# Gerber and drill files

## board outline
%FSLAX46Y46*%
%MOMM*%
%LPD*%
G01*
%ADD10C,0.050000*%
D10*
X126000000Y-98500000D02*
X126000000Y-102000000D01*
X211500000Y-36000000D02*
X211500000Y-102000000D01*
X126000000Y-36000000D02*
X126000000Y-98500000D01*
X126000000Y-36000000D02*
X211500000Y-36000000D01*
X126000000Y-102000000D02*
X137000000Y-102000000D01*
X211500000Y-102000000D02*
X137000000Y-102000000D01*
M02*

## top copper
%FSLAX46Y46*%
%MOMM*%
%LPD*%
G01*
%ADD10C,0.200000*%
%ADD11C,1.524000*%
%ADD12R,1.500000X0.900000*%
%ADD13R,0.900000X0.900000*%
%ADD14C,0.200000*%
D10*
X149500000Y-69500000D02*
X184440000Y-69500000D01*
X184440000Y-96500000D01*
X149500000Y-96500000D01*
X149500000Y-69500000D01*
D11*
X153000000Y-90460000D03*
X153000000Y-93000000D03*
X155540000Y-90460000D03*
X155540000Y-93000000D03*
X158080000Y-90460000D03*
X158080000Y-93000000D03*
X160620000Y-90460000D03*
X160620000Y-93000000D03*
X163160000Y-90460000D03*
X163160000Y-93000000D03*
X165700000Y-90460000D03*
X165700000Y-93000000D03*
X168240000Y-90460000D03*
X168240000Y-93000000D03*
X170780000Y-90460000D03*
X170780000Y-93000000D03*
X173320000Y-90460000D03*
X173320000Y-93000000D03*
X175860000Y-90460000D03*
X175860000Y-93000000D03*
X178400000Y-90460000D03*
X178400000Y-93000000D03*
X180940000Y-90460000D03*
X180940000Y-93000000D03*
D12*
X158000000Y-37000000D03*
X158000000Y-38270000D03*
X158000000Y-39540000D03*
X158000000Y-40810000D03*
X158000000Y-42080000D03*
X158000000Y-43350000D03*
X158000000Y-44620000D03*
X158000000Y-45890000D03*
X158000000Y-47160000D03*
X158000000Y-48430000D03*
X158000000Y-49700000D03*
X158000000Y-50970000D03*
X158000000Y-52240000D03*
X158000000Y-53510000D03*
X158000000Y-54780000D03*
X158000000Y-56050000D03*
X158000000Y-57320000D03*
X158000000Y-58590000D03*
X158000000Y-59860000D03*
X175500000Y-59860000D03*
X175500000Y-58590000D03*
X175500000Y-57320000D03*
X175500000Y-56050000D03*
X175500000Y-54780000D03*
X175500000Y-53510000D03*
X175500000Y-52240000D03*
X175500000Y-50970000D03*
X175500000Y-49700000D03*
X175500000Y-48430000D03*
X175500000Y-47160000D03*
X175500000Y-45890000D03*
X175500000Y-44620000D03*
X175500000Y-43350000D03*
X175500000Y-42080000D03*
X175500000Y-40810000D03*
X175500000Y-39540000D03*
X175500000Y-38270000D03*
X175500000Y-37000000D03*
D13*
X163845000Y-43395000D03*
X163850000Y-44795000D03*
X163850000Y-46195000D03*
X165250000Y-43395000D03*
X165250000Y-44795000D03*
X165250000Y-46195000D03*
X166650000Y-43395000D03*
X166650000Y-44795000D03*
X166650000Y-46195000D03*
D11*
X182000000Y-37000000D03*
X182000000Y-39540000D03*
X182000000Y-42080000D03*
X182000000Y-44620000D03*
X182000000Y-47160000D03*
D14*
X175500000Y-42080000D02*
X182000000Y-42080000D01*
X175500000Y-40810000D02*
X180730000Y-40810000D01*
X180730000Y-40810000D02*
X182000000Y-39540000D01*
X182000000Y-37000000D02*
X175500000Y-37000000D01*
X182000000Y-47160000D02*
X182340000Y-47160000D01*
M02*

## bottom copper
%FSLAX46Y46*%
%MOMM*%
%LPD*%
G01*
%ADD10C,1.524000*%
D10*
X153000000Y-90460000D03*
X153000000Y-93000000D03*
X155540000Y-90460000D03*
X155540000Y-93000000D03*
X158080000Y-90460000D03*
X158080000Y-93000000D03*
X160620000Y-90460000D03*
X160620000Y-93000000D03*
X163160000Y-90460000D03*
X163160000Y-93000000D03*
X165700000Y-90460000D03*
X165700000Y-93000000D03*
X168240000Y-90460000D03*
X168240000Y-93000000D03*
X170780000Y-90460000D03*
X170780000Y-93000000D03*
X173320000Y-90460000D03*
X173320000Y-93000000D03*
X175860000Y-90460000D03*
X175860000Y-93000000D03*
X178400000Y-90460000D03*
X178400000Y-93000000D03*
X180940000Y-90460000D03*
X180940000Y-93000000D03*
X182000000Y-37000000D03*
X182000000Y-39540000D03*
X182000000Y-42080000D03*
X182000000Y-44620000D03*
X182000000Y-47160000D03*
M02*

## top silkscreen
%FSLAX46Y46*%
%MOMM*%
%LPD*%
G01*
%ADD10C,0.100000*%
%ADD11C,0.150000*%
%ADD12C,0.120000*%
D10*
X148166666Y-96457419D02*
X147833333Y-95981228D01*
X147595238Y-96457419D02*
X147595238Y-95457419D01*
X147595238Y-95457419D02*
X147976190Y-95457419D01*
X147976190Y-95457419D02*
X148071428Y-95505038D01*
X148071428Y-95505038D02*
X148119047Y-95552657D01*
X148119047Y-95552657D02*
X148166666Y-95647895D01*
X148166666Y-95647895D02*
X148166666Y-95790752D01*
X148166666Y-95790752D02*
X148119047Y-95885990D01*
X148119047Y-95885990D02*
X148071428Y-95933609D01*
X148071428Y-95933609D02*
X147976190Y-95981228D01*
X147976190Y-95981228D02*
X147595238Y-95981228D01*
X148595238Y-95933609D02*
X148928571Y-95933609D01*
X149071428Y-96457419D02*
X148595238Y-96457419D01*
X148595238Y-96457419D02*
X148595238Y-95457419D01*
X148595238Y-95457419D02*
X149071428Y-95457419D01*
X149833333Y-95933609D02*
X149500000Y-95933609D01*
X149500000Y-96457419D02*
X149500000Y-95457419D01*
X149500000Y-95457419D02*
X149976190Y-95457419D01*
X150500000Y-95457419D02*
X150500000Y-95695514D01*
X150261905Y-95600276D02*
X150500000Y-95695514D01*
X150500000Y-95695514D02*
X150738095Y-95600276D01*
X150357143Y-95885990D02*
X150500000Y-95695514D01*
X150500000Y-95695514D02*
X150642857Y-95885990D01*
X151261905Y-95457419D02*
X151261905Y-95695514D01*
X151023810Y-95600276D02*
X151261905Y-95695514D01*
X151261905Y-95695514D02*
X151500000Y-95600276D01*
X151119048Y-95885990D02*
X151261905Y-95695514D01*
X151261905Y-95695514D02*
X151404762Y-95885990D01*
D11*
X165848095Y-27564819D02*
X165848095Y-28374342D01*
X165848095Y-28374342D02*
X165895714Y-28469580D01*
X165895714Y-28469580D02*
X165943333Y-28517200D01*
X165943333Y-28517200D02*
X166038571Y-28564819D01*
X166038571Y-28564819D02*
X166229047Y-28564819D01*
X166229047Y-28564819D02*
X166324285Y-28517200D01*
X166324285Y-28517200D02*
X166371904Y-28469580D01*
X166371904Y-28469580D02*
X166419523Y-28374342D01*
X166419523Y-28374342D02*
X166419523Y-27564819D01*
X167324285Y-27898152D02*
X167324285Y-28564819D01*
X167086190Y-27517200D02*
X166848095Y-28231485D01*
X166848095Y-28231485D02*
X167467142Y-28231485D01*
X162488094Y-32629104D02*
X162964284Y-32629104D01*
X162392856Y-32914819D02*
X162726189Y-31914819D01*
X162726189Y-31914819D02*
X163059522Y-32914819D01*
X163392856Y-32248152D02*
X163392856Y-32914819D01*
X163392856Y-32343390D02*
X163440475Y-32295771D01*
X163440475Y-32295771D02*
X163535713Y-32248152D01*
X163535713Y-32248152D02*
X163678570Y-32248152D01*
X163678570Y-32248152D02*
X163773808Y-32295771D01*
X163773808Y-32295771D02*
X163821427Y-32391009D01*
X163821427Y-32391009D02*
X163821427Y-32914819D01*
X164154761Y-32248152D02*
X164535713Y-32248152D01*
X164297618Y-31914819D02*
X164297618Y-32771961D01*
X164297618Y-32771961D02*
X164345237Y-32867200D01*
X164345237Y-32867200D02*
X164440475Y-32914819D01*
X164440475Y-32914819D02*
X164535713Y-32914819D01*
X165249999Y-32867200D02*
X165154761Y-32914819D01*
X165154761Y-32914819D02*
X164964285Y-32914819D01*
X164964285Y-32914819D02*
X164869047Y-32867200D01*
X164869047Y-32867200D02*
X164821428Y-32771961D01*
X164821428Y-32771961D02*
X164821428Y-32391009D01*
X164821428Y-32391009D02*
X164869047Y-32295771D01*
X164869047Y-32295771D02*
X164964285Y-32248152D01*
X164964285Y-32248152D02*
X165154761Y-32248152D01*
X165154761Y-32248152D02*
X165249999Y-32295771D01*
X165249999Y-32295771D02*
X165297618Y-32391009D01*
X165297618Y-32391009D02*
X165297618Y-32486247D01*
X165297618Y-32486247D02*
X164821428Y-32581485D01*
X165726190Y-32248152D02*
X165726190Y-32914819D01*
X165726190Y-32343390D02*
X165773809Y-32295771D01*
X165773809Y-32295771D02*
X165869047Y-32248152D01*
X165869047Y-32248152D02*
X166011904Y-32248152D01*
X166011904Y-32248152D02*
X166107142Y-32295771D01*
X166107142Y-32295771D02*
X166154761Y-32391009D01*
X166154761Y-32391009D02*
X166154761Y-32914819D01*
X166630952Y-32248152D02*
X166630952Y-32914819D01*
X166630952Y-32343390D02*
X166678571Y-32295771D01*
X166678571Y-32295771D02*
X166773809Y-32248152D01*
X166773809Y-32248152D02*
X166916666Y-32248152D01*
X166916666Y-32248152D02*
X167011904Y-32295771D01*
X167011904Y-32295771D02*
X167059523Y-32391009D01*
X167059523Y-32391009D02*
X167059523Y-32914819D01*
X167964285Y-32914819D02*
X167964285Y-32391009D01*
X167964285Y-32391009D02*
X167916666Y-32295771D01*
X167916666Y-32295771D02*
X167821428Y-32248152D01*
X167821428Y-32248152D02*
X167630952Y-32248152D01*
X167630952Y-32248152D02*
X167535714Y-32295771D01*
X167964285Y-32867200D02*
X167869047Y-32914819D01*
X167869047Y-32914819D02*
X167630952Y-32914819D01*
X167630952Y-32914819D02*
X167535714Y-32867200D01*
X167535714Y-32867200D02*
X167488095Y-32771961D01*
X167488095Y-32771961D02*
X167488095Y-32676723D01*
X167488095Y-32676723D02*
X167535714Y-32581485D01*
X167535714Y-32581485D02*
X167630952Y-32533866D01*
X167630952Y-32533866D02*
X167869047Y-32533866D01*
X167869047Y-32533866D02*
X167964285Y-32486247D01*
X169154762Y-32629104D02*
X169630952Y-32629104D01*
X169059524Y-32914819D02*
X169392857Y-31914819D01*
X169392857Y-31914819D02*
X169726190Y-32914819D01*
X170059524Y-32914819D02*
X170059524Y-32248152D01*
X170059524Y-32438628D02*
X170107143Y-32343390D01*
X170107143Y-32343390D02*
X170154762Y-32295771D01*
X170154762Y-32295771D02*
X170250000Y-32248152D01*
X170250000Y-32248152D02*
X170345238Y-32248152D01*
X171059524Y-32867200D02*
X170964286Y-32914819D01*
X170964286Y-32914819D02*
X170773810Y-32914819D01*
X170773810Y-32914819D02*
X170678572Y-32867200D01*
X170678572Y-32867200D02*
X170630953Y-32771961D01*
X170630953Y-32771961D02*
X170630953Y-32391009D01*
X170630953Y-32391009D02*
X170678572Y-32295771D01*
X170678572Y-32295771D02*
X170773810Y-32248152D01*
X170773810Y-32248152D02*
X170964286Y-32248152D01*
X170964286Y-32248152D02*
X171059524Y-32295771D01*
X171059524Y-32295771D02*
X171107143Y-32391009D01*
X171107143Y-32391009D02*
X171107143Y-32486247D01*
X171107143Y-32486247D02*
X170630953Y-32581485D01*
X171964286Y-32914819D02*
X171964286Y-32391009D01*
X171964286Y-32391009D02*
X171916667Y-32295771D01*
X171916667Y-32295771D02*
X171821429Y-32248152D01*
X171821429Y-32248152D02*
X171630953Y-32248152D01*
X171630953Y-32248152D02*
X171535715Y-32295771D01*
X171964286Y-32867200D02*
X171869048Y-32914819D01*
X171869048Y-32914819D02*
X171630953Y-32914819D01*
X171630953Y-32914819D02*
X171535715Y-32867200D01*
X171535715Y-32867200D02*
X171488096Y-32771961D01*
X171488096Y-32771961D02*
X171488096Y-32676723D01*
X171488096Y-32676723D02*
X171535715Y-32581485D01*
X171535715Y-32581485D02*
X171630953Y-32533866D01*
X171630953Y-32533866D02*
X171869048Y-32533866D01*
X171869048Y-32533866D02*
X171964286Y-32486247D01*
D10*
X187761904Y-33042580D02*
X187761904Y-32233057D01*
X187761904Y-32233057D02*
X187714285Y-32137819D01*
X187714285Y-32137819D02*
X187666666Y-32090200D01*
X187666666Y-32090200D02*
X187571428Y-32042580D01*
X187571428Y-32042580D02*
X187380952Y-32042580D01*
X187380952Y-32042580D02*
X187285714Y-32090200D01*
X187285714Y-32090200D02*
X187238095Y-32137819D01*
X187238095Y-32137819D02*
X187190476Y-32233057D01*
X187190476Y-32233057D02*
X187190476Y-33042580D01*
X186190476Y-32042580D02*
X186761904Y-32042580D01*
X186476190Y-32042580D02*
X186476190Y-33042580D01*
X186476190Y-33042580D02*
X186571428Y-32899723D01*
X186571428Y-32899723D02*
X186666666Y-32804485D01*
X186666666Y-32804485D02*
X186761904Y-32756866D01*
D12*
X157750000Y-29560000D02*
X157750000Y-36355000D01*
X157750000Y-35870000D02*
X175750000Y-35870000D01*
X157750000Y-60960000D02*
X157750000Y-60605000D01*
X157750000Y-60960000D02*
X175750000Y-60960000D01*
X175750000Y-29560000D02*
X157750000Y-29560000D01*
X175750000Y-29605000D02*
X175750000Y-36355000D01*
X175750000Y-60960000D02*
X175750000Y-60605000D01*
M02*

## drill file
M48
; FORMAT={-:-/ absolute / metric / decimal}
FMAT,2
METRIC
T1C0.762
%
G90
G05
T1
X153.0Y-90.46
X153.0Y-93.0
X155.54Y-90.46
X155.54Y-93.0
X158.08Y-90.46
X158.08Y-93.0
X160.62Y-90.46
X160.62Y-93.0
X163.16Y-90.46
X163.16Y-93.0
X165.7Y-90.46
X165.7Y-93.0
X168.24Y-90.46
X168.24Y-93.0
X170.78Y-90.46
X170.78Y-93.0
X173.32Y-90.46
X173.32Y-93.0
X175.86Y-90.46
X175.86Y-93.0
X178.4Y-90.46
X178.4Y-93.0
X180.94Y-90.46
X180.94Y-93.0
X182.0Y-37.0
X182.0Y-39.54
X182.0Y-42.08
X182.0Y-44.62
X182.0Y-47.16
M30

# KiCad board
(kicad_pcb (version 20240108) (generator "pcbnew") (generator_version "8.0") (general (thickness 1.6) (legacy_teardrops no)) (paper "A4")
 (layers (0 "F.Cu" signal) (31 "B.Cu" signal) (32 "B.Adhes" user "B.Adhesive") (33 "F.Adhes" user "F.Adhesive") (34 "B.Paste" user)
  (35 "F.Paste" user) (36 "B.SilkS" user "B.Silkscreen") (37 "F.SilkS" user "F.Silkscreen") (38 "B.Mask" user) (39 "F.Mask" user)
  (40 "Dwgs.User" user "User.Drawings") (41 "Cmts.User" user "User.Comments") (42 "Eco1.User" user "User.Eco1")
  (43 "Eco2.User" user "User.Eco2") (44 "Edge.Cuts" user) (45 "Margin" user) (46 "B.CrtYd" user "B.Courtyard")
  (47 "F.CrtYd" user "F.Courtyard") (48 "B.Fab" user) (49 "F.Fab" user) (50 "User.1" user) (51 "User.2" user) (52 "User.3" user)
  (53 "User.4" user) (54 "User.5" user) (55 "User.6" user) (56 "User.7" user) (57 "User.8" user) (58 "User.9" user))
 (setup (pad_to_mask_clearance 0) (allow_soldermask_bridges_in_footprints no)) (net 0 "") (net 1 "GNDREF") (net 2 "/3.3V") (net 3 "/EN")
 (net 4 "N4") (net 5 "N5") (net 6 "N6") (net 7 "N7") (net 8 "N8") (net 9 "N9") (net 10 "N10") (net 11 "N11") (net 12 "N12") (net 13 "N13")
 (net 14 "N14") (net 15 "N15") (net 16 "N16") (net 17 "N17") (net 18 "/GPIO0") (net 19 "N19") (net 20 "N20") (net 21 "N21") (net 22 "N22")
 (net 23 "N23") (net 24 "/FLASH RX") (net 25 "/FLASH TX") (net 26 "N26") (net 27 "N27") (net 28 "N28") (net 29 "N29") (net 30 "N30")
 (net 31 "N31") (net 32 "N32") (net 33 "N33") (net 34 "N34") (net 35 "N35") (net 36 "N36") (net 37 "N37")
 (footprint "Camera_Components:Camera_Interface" (layer "F.Cu") (at 149.5 96.5)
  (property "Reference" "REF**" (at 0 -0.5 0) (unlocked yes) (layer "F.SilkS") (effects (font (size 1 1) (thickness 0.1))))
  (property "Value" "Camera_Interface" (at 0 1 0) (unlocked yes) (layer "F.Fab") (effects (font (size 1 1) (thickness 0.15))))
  (fp_rect (start 0 0) (end 34.94 -27) (stroke (width 0.2) (type default)) (fill none) (layer "F.Cu"))
  (pad "1" thru_hole circle (at 3.5 -6.04 270) (size 1.524 1.524) (drill 0.762) (layers "*.Cu" "*.Mask") (remove_unused_layers no))
  (pad "2" thru_hole circle (at 3.5 -3.5 270) (size 1.524 1.524) (drill 0.762) (layers "*.Cu" "*.Mask") (remove_unused_layers no))
  (pad "3" thru_hole circle (at 6.04 -6.04 270) (size 1.524 1.524) (drill 0.762) (layers "*.Cu" "*.Mask") (remove_unused_layers no))
  (pad "4" thru_hole circle (at 6.04 -3.5 270) (size 1.524 1.524) (drill 0.762) (layers "*.Cu" "*.Mask") (remove_unused_layers no))
  (pad "5" thru_hole circle (at 8.58 -6.04 270) (size 1.524 1.524) (drill 0.762) (layers "*.Cu" "*.Mask") (remove_unused_layers no))
  (pad "6" thru_hole circle (at 8.58 -3.5 270) (size 1.524 1.524) (drill 0.762) (layers "*.Cu" "*.Mask") (remove_unused_layers no))
  (pad "7" thru_hole circle (at 11.12 -6.04 270) (size 1.524 1.524) (drill 0.762) (layers "*.Cu" "*.Mask") (remove_unused_layers no))
  (pad "8" thru_hole circle (at 11.12 -3.5 270) (size 1.524 1.524) (drill 0.762) (layers "*.Cu" "*.Mask") (remove_unused_layers no))
  (pad "9" thru_hole circle (at 13.66 -6.04 270) (size 1.524 1.524) (drill 0.762) (layers "*.Cu" "*.Mask") (remove_unused_layers no))
  (pad "10" thru_hole circle (at 13.66 -3.5 270) (size 1.524 1.524) (drill 0.762) (layers "*.Cu" "*.Mask") (remove_unused_layers no))
  (pad "11" thru_hole circle (at 16.2 -6.04 270) (size 1.524 1.524) (drill 0.762) (layers "*.Cu" "*.Mask") (remove_unused_layers no))
  (pad "12" thru_hole circle (at 16.2 -3.5 270) (size 1.524 1.524) (drill 0.762) (layers "*.Cu" "*.Mask") (remove_unused_layers no))
  (pad "13" thru_hole circle (at 18.74 -6.04 270) (size 1.524 1.524) (drill 0.762) (layers "*.Cu" "*.Mask") (remove_unused_layers no))
  (pad "14" thru_hole circle (at 18.74 -3.5 270) (size 1.524 1.524) (drill 0.762) (layers "*.Cu" "*.Mask") (remove_unused_layers no))
  (pad "15" thru_hole circle (at 21.28 -6.04 270) (size 1.524 1.524) (drill 0.762) (layers "*.Cu" "*.Mask") (remove_unused_layers no))
  (pad "16" thru_hole circle (at 21.28 -3.5 270) (size 1.524 1.524) (drill 0.762) (layers "*.Cu" "*.Mask") (remove_unused_layers no))
  (pad "17" thru_hole circle (at 23.82 -6.04 270) (size 1.524 1.524) (drill 0.762) (layers "*.Cu" "*.Mask") (remove_unused_layers no))
  (pad "18" thru_hole circle (at 23.82 -3.5 270) (size 1.524 1.524) (drill 0.762) (layers "*.Cu" "*.Mask") (remove_unused_layers no))
  (pad "19" thru_hole circle (at 26.36 -6.04 270) (size 1.524 1.524) (drill 0.762) (layers "*.Cu" "*.Mask") (remove_unused_layers no))
  (pad "20" thru_hole circle (at 26.36 -3.5 270) (size 1.524 1.524) (drill 0.762) (layers "*.Cu" "*.Mask") (remove_unused_layers no))
  (pad "21" thru_hole circle (at 28.9 -6.04 270) (size 1.524 1.524) (drill 0.762) (layers "*.Cu" "*.Mask") (remove_unused_layers no))
  (pad "22" thru_hole circle (at 28.9 -3.5 270) (size 1.524 1.524) (drill 0.762) (layers "*.Cu" "*.Mask") (remove_unused_layers no))
  (pad "23" thru_hole circle (at 31.44 -6.04 270) (size 1.524 1.524) (drill 0.762) (layers "*.Cu" "*.Mask") (remove_unused_layers no))
  (pad "24" thru_hole circle (at 31.44 -3.5 270) (size 1.524 1.524) (drill 0.762) (layers "*.Cu" "*.Mask") (remove_unused_layers no)))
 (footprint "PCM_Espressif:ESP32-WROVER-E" (layer "F.Cu") (at 166.75 45.255)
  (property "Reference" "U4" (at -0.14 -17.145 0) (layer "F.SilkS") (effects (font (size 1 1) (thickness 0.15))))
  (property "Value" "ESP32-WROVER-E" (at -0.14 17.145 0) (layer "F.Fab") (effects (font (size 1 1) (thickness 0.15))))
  (fp_line (start -9 -15.695) (end -9 -8.9) (stroke (width 0.12) (type solid)) (layer "F.SilkS"))
  (fp_line (start -9 -9.385) (end 9 -9.385) (stroke (width 0.12) (type solid)) (layer "F.SilkS"))
  (fp_line (start -9 15.705) (end -9 15.35) (stroke (width 0.12) (type solid)) (layer "F.SilkS"))
  (fp_line (start -9 15.705) (end 9 15.705) (stroke (width 0.12) (type solid)) (layer "F.SilkS"))
  (fp_line (start 9 -15.695) (end -9 -15.695) (stroke (width 0.12) (type solid)) (layer "F.SilkS"))
  (fp_line (start 9 -15.65) (end 9 -8.9) (stroke (width 0.12) (type solid)) (layer "F.SilkS"))
  (fp_line (start 9 15.705) (end 9 15.35) (stroke (width 0.12) (type solid)) (layer "F.SilkS"))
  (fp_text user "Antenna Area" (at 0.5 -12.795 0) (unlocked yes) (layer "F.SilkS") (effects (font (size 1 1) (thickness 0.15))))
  (pad "1" smd rect (at -8.75 -8.255) (size 1.5 0.9) (layers "F.Cu" "F.Paste" "F.Mask") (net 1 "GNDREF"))
  (pad "2" smd rect (at -8.75 -6.985) (size 1.5 0.9) (layers "F.Cu" "F.Paste" "F.Mask") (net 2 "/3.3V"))
  (pad "3" smd rect (at -8.75 -5.715) (size 1.5 0.9) (layers "F.Cu" "F.Paste" "F.Mask") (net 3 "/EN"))
  (pad "4" smd rect (at -8.75 -4.445) (size 1.5 0.9) (layers "F.Cu" "F.Paste" "F.Mask") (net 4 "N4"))
  (pad "5" smd rect (at -8.75 -3.175) (size 1.5 0.9) (layers "F.Cu" "F.Paste" "F.Mask") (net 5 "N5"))
  (pad "6" smd rect (at -8.75 -1.905) (size 1.5 0.9) (layers "F.Cu" "F.Paste" "F.Mask") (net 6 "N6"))
  (pad "7" smd rect (at -8.75 -0.635) (size 1.5 0.9) (layers "F.Cu" "F.Paste" "F.Mask") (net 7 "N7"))
  (pad "8" smd rect (at -8.75 0.635) (size 1.5 0.9) (layers "F.Cu" "F.Paste" "F.Mask") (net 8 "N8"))
  (pad "9" smd rect (at -8.75 1.905) (size 1.5 0.9) (layers "F.Cu" "F.Paste" "F.Mask") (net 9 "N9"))
  (pad "10" smd rect (at -8.75 3.175) (size 1.5 0.9) (layers "F.Cu" "F.Paste" "F.Mask") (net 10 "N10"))
  (pad "11" smd rect (at -8.75 4.445) (size 1.5 0.9) (layers "F.Cu" "F.Paste" "F.Mask") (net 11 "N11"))
  (pad "12" smd rect (at -8.75 5.715) (size 1.5 0.9) (layers "F.Cu" "F.Paste" "F.Mask") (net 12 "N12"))
  (pad "13" smd rect (at -8.75 6.985) (size 1.5 0.9) (layers "F.Cu" "F.Paste" "F.Mask") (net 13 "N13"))
  (pad "14" smd rect (at -8.75 8.255) (size 1.5 0.9) (layers "F.Cu" "F.Paste" "F.Mask") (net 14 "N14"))
  (pad "15" smd rect (at -8.75 9.525) (size 1.5 0.9) (layers "F.Cu" "F.Paste" "F.Mask") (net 1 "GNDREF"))
  (pad "16" smd rect (at -8.75 10.795) (size 1.5 0.9) (layers "F.Cu" "F.Paste" "F.Mask") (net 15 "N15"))
  (pad "17" smd rect (at -8.75 12.065) (size 1.5 0.9) (layers "F.Cu" "F.Paste" "F.Mask"))
  (pad "18" smd rect (at -8.75 13.335) (size 1.5 0.9) (layers "F.Cu" "F.Paste" "F.Mask"))
  (pad "19" smd rect (at -8.75 14.605) (size 1.5 0.9) (layers "F.Cu" "F.Paste" "F.Mask"))
  (pad "20" smd rect (at 8.75 14.605) (size 1.5 0.9) (layers "F.Cu" "F.Paste" "F.Mask"))
  (pad "21" smd rect (at 8.75 13.335) (size 1.5 0.9) (layers "F.Cu" "F.Paste" "F.Mask"))
  (pad "22" smd rect (at 8.75 12.065) (size 1.5 0.9) (layers "F.Cu" "F.Paste" "F.Mask"))
  (pad "23" smd rect (at 8.75 10.795) (size 1.5 0.9) (layers "F.Cu" "F.Paste" "F.Mask") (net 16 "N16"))
  (pad "24" smd rect (at 8.75 9.525) (size 1.5 0.9) (layers "F.Cu" "F.Paste" "F.Mask") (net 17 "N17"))
  (pad "25" smd rect (at 8.75 8.255) (size 1.5 0.9) (layers "F.Cu" "F.Paste" "F.Mask") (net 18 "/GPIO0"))
  (pad "26" smd rect (at 8.75 6.985) (size 1.5 0.9) (layers "F.Cu" "F.Paste" "F.Mask") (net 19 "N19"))
  (pad "27" smd rect (at 8.75 5.715) (size 1.5 0.9) (layers "F.Cu" "F.Paste" "F.Mask"))
  (pad "28" smd rect (at 8.75 4.445) (size 1.5 0.9) (layers "F.Cu" "F.Paste" "F.Mask"))
  (pad "29" smd rect (at 8.75 3.175) (size 1.5 0.9) (layers "F.Cu" "F.Paste" "F.Mask") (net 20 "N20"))
  (pad "30" smd rect (at 8.75 1.905) (size 1.5 0.9) (layers "F.Cu" "F.Paste" "F.Mask") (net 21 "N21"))
  (pad "31" smd rect (at 8.75 0.635) (size 1.5 0.9) (layers "F.Cu" "F.Paste" "F.Mask") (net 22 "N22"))
  (pad "32" smd rect (at 8.75 -0.635) (size 1.5 0.9) (layers "F.Cu" "F.Paste" "F.Mask"))
  (pad "33" smd rect (at 8.75 -1.905) (size 1.5 0.9) (layers "F.Cu" "F.Paste" "F.Mask") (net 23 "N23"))
  (pad "34" smd rect (at 8.75 -3.175) (size 1.5 0.9) (layers "F.Cu" "F.Paste" "F.Mask") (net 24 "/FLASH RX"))
  (pad "35" smd rect (at 8.75 -4.445) (size 1.5 0.9) (layers "F.Cu" "F.Paste" "F.Mask") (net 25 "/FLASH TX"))
  (pad "36" smd rect (at 8.75 -5.715) (size 1.5 0.9) (layers "F.Cu" "F.Paste" "F.Mask") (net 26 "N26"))
  (pad "37" smd rect (at 8.75 -6.985) (size 1.5 0.9) (layers "F.Cu" "F.Paste" "F.Mask") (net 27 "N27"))
  (pad "38" smd rect (at 8.75 -8.255) (size 1.5 0.9) (layers "F.Cu" "F.Paste" "F.Mask") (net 1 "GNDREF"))
  (pad "39" smd rect (at -2.905 -1.86) (size 0.9 0.9) (layers "F.Cu" "F.Paste" "F.Mask") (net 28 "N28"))
  (pad "39" smd rect (at -2.9 -0.46) (size 0.9 0.9) (layers "F.Cu" "F.Paste" "F.Mask") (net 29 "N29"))
  (pad "39" smd rect (at -2.9 0.94) (size 0.9 0.9) (layers "F.Cu" "F.Paste" "F.Mask") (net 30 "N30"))
  (pad "39" smd rect (at -1.5 -1.86) (size 0.9 0.9) (layers "F.Cu" "F.Paste" "F.Mask") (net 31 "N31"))
  (pad "39" smd rect (at -1.5 -0.46) (size 0.9 0.9) (layers "F.Cu" "F.Paste" "F.Mask") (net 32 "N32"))
  (pad "39" smd rect (at -1.5 0.94) (size 0.9 0.9) (layers "F.Cu" "F.Paste" "F.Mask") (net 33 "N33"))
  (pad "39" smd rect (at -0.1 -1.86) (size 0.9 0.9) (layers "F.Cu" "F.Paste" "F.Mask") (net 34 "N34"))
  (pad "39" smd rect (at -0.1 -0.46) (size 0.9 0.9) (layers "F.Cu" "F.Paste" "F.Mask") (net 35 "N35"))
  (pad "39" smd rect (at -0.1 0.94) (size 0.9 0.9) (layers "F.Cu" "F.Paste" "F.Mask") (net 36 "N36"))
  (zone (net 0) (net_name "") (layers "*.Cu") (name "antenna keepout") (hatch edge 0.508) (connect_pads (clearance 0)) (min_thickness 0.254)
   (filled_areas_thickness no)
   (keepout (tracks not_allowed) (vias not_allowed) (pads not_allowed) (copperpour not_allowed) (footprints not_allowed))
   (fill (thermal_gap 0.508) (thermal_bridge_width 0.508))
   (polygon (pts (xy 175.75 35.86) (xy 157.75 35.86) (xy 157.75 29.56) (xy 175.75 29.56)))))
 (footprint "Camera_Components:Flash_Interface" (layer "F.Cu") (at 187 32 180)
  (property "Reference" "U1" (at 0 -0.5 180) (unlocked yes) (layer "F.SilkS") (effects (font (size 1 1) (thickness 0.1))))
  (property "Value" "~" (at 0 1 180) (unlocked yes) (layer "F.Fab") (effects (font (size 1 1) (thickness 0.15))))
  (pad "1" thru_hole circle (at 5 -5 180) (size 1.524 1.524) (drill 0.762) (layers "*.Cu" "*.Mask") (remove_unused_layers no)
   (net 1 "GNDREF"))
  (pad "2" thru_hole circle (at 5 -7.54 180) (size 1.524 1.524) (drill 0.762) (layers "*.Cu" "*.Mask") (remove_unused_layers no)
   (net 25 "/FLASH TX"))
  (pad "3" thru_hole circle (at 5 -10.08 180) (size 1.524 1.524) (drill 0.762) (layers "*.Cu" "*.Mask") (remove_unused_layers no)
   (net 24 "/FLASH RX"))
  (pad "4" thru_hole circle (at 5 -12.62 180) (size 1.524 1.524) (drill 0.762) (layers "*.Cu" "*.Mask") (remove_unused_layers no)
   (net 2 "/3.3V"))
  (pad "5" thru_hole circle (at 5 -15.16 180) (size 1.524 1.524) (drill 0.762) (layers "*.Cu" "*.Mask") (remove_unused_layers no)
   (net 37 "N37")))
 (gr_line (start 126 98.5) (end 126 102) (stroke (width 0.05) (type default)) (layer "Edge.Cuts"))
 (gr_line (start 211.5 36) (end 211.5 102) (stroke (width 0.05) (type default)) (layer "Edge.Cuts"))
 (gr_line (start 126 36) (end 126 98.5) (stroke (width 0.05) (type default)) (layer "Edge.Cuts"))
 (gr_line (start 126 36) (end 211.5 36) (stroke (width 0.05) (type default)) (layer "Edge.Cuts"))
 (gr_line (start 126 102) (end 137 102) (stroke (width 0.05) (type default)) (layer "Edge.Cuts"))
 (gr_line (start 211.5 102) (end 137 102) (stroke (width 0.05) (type default)) (layer "Edge.Cuts"))
 (segment (start 175.5 42.08) (end 182 42.08) (width 0.2) (layer "F.Cu") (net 24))
 (segment (start 175.5 40.81) (end 180.73 40.81) (width 0.2) (layer "F.Cu") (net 25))
 (segment (start 180.73 40.81) (end 182 39.54) (width 0.2) (layer "F.Cu") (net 25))
 (segment (start 182 37) (end 175.5 37) (width 0.2) (layer "F.Cu") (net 1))
 (segment (start 182 47.16) (end 182.34 47.16) (width 0.2) (layer "F.Cu") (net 37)))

